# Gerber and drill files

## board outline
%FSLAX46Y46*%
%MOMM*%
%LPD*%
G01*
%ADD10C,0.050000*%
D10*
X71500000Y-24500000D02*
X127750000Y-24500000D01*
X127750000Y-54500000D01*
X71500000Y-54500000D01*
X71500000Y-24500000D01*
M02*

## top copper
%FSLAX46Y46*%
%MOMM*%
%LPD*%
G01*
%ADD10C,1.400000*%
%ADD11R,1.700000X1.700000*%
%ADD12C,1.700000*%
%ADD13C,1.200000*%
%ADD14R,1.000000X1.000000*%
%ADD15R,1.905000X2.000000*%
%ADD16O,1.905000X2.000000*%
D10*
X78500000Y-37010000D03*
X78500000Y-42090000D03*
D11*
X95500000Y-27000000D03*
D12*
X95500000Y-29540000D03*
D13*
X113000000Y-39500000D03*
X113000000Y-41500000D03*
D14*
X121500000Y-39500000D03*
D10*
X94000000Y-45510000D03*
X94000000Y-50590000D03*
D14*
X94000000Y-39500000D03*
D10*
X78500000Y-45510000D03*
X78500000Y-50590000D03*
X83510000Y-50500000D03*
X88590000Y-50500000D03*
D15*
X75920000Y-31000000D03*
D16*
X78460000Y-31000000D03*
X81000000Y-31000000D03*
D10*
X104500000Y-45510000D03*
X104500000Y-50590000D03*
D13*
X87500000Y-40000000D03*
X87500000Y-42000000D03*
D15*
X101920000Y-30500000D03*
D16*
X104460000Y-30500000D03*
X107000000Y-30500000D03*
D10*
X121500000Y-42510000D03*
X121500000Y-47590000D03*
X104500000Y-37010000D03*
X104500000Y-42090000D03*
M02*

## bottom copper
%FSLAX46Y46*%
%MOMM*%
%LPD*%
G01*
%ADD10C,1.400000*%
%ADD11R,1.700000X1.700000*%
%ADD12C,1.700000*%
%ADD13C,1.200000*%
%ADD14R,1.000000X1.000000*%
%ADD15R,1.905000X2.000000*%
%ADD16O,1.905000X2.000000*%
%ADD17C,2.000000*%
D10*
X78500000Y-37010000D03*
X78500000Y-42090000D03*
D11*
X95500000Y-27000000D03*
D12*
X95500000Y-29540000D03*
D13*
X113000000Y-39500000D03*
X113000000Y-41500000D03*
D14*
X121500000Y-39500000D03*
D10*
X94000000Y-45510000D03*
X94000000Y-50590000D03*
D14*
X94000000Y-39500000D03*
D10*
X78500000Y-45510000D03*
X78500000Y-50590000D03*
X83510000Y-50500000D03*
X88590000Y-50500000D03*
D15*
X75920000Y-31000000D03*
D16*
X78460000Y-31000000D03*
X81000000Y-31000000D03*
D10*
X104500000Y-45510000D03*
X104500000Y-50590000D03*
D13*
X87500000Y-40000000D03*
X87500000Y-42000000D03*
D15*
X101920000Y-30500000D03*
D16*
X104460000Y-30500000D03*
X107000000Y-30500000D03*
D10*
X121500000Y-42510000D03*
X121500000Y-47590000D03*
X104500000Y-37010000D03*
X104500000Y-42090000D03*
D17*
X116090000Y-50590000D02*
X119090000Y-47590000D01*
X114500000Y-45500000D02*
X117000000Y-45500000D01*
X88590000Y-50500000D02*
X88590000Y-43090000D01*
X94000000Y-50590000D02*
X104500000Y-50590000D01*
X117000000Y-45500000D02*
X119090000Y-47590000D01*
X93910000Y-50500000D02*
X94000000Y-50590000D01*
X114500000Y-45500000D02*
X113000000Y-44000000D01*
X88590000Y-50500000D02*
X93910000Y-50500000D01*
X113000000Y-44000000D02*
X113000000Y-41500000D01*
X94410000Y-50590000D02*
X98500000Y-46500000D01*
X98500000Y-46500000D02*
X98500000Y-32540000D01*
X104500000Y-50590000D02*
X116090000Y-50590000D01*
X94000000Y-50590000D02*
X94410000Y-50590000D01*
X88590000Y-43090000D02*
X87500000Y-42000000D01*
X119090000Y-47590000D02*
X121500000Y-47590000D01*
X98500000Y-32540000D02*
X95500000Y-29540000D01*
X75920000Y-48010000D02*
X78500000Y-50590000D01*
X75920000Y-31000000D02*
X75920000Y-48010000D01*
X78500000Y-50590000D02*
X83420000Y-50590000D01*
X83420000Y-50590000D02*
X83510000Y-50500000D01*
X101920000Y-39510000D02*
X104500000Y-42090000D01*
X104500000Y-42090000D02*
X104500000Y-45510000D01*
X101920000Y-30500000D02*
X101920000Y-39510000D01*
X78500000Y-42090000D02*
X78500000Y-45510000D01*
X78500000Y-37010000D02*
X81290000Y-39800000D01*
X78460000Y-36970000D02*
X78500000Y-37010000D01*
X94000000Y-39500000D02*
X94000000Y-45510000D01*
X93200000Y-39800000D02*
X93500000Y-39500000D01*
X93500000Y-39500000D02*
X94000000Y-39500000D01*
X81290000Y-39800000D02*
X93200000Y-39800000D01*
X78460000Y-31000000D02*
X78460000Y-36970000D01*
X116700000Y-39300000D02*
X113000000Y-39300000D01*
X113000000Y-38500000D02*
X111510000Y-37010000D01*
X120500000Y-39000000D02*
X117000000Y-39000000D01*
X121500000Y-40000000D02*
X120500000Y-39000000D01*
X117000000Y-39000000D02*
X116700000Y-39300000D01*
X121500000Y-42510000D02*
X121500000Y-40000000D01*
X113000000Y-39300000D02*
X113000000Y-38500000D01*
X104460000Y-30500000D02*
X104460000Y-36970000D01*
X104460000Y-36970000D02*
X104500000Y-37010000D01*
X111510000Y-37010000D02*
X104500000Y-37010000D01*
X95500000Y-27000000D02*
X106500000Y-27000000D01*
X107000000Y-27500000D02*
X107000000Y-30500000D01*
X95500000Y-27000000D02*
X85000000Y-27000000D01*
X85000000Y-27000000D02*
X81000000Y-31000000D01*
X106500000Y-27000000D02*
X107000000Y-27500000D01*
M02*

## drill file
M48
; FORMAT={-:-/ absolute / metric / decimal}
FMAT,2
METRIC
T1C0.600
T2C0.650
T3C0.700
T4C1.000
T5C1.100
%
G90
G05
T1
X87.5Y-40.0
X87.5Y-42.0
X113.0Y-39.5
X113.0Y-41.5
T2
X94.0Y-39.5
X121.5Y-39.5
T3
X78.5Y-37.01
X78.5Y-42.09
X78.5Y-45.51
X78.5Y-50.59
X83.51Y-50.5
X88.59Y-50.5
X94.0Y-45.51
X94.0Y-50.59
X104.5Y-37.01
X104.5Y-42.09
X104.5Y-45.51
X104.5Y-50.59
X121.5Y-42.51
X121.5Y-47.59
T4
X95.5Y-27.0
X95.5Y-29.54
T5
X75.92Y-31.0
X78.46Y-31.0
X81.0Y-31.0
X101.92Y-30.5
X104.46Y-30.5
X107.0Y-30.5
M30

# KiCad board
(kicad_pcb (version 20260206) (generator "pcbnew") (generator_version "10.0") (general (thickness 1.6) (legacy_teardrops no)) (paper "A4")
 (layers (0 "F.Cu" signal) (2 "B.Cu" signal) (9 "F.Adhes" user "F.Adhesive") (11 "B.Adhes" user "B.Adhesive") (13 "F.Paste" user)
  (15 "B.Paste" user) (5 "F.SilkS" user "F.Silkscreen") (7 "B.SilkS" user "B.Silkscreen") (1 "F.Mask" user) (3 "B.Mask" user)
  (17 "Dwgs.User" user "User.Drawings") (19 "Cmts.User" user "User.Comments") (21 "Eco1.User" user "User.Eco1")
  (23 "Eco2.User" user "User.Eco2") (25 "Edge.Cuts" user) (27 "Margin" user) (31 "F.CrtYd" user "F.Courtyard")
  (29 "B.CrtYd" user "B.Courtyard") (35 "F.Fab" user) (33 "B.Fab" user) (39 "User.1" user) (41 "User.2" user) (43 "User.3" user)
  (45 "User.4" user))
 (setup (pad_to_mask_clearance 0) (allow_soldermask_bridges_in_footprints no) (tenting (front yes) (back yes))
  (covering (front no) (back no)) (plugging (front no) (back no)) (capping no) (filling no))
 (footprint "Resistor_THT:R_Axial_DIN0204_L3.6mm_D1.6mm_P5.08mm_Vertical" (layer "F.Cu") (at 78.5 37.01 -90)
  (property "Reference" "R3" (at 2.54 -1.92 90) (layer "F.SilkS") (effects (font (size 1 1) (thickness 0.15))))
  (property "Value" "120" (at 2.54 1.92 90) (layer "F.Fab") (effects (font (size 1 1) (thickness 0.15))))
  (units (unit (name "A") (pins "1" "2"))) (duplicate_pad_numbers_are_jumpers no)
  (pad "1" thru_hole circle (at 0 0 270) (size 1.4 1.4) (drill 0.7) (layers "*.Cu" "*.Mask") (remove_unused_layers no)
   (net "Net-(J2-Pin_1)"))
  (pad "2" thru_hole circle (at 5.08 0 270) (size 1.4 1.4) (drill 0.7) (layers "*.Cu" "*.Mask") (remove_unused_layers no)
   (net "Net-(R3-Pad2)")))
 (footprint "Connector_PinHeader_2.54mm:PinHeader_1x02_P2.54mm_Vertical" (layer "F.Cu") (at 95.5 27)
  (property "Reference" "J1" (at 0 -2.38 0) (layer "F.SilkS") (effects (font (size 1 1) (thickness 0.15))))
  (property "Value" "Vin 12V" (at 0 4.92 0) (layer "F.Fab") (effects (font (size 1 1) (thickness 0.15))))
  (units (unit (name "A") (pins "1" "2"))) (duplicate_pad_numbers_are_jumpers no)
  (pad "1" thru_hole rect (at 0 0) (size 1.7 1.7) (drill 1) (layers "*.Cu" "*.Mask") (remove_unused_layers no) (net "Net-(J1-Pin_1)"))
  (pad "2" thru_hole circle (at 0 2.54) (size 1.7 1.7) (drill 1) (layers "*.Cu" "*.Mask") (remove_unused_layers no) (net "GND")))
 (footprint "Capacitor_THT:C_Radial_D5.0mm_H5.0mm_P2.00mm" (layer "F.Cu") (at 113 39.5 -90)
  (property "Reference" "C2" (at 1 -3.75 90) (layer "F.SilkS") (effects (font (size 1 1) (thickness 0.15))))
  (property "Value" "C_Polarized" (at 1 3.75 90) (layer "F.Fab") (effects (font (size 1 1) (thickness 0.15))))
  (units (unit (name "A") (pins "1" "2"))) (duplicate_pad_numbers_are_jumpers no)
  (pad "1" thru_hole circle (at 0 0 270) (size 1.2 1.2) (drill 0.6) (layers "*.Cu" "*.Mask") (remove_unused_layers no)
   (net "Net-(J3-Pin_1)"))
  (pad "2" thru_hole circle (at 2 0 270) (size 1.2 1.2) (drill 0.6) (layers "*.Cu" "*.Mask") (remove_unused_layers no) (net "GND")))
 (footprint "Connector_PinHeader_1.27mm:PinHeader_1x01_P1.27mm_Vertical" (layer "F.Cu") (at 121.5 39.5)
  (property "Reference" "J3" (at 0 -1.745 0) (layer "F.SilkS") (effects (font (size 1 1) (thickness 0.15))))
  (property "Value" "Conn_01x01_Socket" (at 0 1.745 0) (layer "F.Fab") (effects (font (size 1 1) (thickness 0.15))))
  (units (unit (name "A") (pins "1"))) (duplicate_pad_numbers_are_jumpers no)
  (pad "1" thru_hole rect (at 0 0) (size 1 1) (drill 0.65) (layers "*.Cu" "*.Mask") (remove_unused_layers no) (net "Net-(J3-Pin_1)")))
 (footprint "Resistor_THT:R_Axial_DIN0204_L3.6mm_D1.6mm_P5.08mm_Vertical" (layer "F.Cu") (at 94 45.51 -90)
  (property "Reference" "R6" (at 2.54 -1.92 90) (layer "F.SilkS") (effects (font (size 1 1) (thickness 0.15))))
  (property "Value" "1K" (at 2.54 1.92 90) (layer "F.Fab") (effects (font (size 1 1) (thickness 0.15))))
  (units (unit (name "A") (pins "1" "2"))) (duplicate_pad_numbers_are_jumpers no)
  (pad "1" thru_hole circle (at 0 0 270) (size 1.4 1.4) (drill 0.7) (layers "*.Cu" "*.Mask") (remove_unused_layers no)
   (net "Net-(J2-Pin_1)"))
  (pad "2" thru_hole circle (at 5.08 0 270) (size 1.4 1.4) (drill 0.7) (layers "*.Cu" "*.Mask") (remove_unused_layers no) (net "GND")))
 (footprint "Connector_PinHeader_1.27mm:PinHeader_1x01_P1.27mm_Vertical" (layer "F.Cu") (at 94 39.5)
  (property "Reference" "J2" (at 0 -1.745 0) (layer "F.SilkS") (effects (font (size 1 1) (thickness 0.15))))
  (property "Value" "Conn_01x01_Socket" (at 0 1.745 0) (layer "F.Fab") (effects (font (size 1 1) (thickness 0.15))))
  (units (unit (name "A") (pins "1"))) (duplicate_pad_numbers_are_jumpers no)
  (pad "1" thru_hole rect (at 0 0) (size 1 1) (drill 0.65) (layers "*.Cu" "*.Mask") (remove_unused_layers no) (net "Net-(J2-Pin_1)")))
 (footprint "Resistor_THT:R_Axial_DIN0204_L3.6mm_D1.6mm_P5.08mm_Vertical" (layer "F.Cu") (at 78.5 45.51 -90)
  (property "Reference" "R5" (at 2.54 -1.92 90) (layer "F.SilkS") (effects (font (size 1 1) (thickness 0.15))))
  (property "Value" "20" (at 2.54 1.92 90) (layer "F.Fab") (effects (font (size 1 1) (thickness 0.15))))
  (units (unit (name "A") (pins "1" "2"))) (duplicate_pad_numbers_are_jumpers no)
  (pad "1" thru_hole circle (at 0 0 270) (size 1.4 1.4) (drill 0.7) (layers "*.Cu" "*.Mask") (remove_unused_layers no) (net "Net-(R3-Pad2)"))
  (pad "2" thru_hole circle (at 5.08 0 270) (size 1.4 1.4) (drill 0.7) (layers "*.Cu" "*.Mask") (remove_unused_layers no)
   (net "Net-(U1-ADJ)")))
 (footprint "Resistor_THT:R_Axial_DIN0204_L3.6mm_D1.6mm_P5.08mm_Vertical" (layer "F.Cu") (at 83.51 50.5)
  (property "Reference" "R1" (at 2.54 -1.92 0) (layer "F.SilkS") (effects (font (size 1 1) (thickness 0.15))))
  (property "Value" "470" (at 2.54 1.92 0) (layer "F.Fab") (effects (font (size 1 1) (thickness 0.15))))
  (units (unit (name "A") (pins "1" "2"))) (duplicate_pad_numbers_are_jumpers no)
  (pad "1" thru_hole circle (at 0 0) (size 1.4 1.4) (drill 0.7) (layers "*.Cu" "*.Mask") (remove_unused_layers no) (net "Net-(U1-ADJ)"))
  (pad "2" thru_hole circle (at 5.08 0) (size 1.4 1.4) (drill 0.7) (layers "*.Cu" "*.Mask") (remove_unused_layers no) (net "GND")))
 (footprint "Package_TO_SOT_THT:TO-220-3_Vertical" (layer "F.Cu") (at 75.92 31)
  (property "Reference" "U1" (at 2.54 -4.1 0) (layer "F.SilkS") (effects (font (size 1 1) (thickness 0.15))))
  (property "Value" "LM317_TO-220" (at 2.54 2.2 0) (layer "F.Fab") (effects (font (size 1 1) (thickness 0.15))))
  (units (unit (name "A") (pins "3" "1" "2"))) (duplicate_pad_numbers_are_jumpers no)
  (pad "1" thru_hole rect (at 0 0) (size 1.905 2) (drill 1.1) (layers "*.Cu" "*.Mask") (remove_unused_layers no) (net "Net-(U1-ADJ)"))
  (pad "2" thru_hole oval (at 2.54 0) (size 1.905 2) (drill 1.1) (layers "*.Cu" "*.Mask") (remove_unused_layers no) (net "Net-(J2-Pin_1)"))
  (pad "3" thru_hole oval (at 5.08 0) (size 1.905 2) (drill 1.1) (layers "*.Cu" "*.Mask") (remove_unused_layers no) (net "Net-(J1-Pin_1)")))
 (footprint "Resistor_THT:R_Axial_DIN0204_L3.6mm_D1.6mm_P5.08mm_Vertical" (layer "F.Cu") (at 104.5 45.51 -90)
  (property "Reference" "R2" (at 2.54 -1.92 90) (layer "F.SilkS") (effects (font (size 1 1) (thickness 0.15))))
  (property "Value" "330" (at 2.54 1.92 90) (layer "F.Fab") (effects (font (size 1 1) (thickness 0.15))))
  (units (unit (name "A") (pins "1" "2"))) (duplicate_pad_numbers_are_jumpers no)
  (pad "1" thru_hole circle (at 0 0 270) (size 1.4 1.4) (drill 0.7) (layers "*.Cu" "*.Mask") (remove_unused_layers no) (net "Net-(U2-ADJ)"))
  (pad "2" thru_hole circle (at 5.08 0 270) (size 1.4 1.4) (drill 0.7) (layers "*.Cu" "*.Mask") (remove_unused_layers no) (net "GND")))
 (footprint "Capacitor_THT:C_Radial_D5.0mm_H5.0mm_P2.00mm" (layer "F.Cu") (at 87.5 40 -90)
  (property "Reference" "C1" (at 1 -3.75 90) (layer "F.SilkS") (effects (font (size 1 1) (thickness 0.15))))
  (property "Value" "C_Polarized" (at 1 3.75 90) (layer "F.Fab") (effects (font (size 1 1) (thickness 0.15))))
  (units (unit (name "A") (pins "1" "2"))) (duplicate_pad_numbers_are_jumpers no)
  (pad "1" thru_hole circle (at 0 0 270) (size 1.2 1.2) (drill 0.6) (layers "*.Cu" "*.Mask") (remove_unused_layers no)
   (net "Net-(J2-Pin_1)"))
  (pad "2" thru_hole circle (at 2 0 270) (size 1.2 1.2) (drill 0.6) (layers "*.Cu" "*.Mask") (remove_unused_layers no) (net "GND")))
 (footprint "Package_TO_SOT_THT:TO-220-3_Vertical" (layer "F.Cu") (at 101.92 30.5)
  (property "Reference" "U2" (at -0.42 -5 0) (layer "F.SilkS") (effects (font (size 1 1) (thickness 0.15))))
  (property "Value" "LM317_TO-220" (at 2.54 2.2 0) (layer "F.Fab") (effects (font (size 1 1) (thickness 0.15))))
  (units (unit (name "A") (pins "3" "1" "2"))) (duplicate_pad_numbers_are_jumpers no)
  (pad "1" thru_hole rect (at 0 0) (size 1.905 2) (drill 1.1) (layers "*.Cu" "*.Mask") (remove_unused_layers no) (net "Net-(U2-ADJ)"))
  (pad "2" thru_hole oval (at 2.54 0) (size 1.905 2) (drill 1.1) (layers "*.Cu" "*.Mask") (remove_unused_layers no) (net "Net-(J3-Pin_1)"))
  (pad "3" thru_hole oval (at 5.08 0) (size 1.905 2) (drill 1.1) (layers "*.Cu" "*.Mask") (remove_unused_layers no) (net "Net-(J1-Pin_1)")))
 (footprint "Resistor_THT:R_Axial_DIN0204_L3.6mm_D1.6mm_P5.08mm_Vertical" (layer "F.Cu") (at 121.5 42.51 -90)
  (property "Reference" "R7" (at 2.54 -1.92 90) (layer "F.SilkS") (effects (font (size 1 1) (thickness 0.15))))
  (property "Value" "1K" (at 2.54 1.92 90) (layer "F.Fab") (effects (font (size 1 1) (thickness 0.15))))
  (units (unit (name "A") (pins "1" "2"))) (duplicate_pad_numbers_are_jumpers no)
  (pad "1" thru_hole circle (at 0 0 270) (size 1.4 1.4) (drill 0.7) (layers "*.Cu" "*.Mask") (remove_unused_layers no)
   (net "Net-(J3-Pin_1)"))
  (pad "2" thru_hole circle (at 5.08 0 270) (size 1.4 1.4) (drill 0.7) (layers "*.Cu" "*.Mask") (remove_unused_layers no) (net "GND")))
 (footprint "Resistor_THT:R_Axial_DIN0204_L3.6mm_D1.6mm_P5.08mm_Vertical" (layer "F.Cu") (at 104.5 37.01 -90)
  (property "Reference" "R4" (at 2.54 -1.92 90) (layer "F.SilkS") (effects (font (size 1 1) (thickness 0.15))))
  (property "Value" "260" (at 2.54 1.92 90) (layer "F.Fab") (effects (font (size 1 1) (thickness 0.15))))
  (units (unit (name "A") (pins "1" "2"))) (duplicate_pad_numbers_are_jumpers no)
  (pad "1" thru_hole circle (at 0 0 270) (size 1.4 1.4) (drill 0.7) (layers "*.Cu" "*.Mask") (remove_unused_layers no)
   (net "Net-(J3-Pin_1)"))
  (pad "2" thru_hole circle (at 5.08 0 270) (size 1.4 1.4) (drill 0.7) (layers "*.Cu" "*.Mask") (remove_unused_layers no)
   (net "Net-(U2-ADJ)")))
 (gr_rect (start 71.5 24.5) (end 127.75 54.5) (stroke (width 0.05) (type default)) (fill no) (layer "Edge.Cuts"))
 (segment (start 116.09 50.59) (end 119.09 47.59) (width 2) (layer "B.Cu") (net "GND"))
 (segment (start 114.5 45.5) (end 117 45.5) (width 2) (layer "B.Cu") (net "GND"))
 (segment (start 88.59 50.5) (end 88.59 43.09) (width 2) (layer "B.Cu") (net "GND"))
 (segment (start 94 50.59) (end 104.5 50.59) (width 2) (layer "B.Cu") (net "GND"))
 (segment (start 117 45.5) (end 119.09 47.59) (width 2) (layer "B.Cu") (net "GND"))
 (segment (start 93.91 50.5) (end 94 50.59) (width 2) (layer "B.Cu") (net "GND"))
 (segment (start 114.5 45.5) (end 113 44) (width 2) (layer "B.Cu") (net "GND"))
 (segment (start 88.59 50.5) (end 93.91 50.5) (width 2) (layer "B.Cu") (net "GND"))
 (segment (start 113 44) (end 113 41.5) (width 2) (layer "B.Cu") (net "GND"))
 (segment (start 94.41 50.59) (end 98.5 46.5) (width 2) (layer "B.Cu") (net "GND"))
 (segment (start 98.5 46.5) (end 98.5 32.54) (width 2) (layer "B.Cu") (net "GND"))
 (segment (start 104.5 50.59) (end 116.09 50.59) (width 2) (layer "B.Cu") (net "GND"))
 (segment (start 94 50.59) (end 94.41 50.59) (width 2) (layer "B.Cu") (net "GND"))
 (segment (start 88.59 43.09) (end 87.5 42) (width 2) (layer "B.Cu") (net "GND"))
 (segment (start 119.09 47.59) (end 121.5 47.59) (width 2) (layer "B.Cu") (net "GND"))
 (segment (start 98.5 32.54) (end 95.5 29.54) (width 2) (layer "B.Cu") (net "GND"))
 (segment (start 75.92 48.01) (end 78.5 50.59) (width 2) (layer "B.Cu") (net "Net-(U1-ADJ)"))
 (segment (start 75.92 31) (end 75.92 48.01) (width 2) (layer "B.Cu") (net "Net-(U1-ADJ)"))
 (segment (start 78.5 50.59) (end 83.42 50.59) (width 2) (layer "B.Cu") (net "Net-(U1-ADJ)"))
 (segment (start 83.42 50.59) (end 83.51 50.5) (width 2) (layer "B.Cu") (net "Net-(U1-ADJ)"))
 (segment (start 101.92 39.51) (end 104.5 42.09) (width 2) (layer "B.Cu") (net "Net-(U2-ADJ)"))
 (segment (start 104.5 42.09) (end 104.5 45.51) (width 2) (layer "B.Cu") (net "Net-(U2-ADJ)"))
 (segment (start 101.92 30.5) (end 101.92 39.51) (width 2) (layer "B.Cu") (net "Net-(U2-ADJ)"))
 (segment (start 78.5 42.09) (end 78.5 45.51) (width 2) (layer "B.Cu") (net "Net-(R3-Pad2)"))
 (segment (start 78.5 37.01) (end 81.29 39.8) (width 2) (layer "B.Cu") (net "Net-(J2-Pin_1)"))
 (segment (start 78.46 36.97) (end 78.5 37.01) (width 2) (layer "B.Cu") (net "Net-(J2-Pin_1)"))
 (segment (start 94 39.5) (end 94 45.51) (width 2) (layer "B.Cu") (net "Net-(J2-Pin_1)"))
 (segment (start 93.2 39.8) (end 93.5 39.5) (width 2) (layer "B.Cu") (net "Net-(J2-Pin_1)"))
 (segment (start 93.5 39.5) (end 94 39.5) (width 2) (layer "B.Cu") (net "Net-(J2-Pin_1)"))
 (segment (start 81.29 39.8) (end 93.2 39.8) (width 2) (layer "B.Cu") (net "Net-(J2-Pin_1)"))
 (segment (start 78.46 31) (end 78.46 36.97) (width 2) (layer "B.Cu") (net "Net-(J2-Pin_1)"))
 (segment (start 116.7 39.3) (end 113 39.3) (width 2) (layer "B.Cu") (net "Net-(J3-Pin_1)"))
 (segment (start 113 38.5) (end 111.51 37.01) (width 2) (layer "B.Cu") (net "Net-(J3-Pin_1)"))
 (segment (start 120.5 39) (end 117 39) (width 2) (layer "B.Cu") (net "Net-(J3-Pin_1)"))
 (segment (start 121.5 40) (end 120.5 39) (width 2) (layer "B.Cu") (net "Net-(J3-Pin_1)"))
 (segment (start 117 39) (end 116.7 39.3) (width 2) (layer "B.Cu") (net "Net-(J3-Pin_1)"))
 (segment (start 121.5 42.51) (end 121.5 40) (width 2) (layer "B.Cu") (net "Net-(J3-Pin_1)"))
 (segment (start 113 39.3) (end 113 38.5) (width 2) (layer "B.Cu") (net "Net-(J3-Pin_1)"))
 (segment (start 104.46 30.5) (end 104.46 36.97) (width 2) (layer "B.Cu") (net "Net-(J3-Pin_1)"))
 (segment (start 104.46 36.97) (end 104.5 37.01) (width 2) (layer "B.Cu") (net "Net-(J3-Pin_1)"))
 (segment (start 111.51 37.01) (end 104.5 37.01) (width 2) (layer "B.Cu") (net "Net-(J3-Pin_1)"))
 (segment (start 95.5 27) (end 106.5 27) (width 2) (layer "B.Cu") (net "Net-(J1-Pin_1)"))
 (segment (start 107 27.5) (end 107 30.5) (width 2) (layer "B.Cu") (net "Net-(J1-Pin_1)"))
 (segment (start 95.5 27) (end 85 27) (width 2) (layer "B.Cu") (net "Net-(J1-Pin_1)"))
 (segment (start 85 27) (end 81 31) (width 2) (layer "B.Cu") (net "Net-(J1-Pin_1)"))
 (segment (start 106.5 27) (end 107 27.5) (width 2) (layer "B.Cu") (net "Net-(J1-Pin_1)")))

